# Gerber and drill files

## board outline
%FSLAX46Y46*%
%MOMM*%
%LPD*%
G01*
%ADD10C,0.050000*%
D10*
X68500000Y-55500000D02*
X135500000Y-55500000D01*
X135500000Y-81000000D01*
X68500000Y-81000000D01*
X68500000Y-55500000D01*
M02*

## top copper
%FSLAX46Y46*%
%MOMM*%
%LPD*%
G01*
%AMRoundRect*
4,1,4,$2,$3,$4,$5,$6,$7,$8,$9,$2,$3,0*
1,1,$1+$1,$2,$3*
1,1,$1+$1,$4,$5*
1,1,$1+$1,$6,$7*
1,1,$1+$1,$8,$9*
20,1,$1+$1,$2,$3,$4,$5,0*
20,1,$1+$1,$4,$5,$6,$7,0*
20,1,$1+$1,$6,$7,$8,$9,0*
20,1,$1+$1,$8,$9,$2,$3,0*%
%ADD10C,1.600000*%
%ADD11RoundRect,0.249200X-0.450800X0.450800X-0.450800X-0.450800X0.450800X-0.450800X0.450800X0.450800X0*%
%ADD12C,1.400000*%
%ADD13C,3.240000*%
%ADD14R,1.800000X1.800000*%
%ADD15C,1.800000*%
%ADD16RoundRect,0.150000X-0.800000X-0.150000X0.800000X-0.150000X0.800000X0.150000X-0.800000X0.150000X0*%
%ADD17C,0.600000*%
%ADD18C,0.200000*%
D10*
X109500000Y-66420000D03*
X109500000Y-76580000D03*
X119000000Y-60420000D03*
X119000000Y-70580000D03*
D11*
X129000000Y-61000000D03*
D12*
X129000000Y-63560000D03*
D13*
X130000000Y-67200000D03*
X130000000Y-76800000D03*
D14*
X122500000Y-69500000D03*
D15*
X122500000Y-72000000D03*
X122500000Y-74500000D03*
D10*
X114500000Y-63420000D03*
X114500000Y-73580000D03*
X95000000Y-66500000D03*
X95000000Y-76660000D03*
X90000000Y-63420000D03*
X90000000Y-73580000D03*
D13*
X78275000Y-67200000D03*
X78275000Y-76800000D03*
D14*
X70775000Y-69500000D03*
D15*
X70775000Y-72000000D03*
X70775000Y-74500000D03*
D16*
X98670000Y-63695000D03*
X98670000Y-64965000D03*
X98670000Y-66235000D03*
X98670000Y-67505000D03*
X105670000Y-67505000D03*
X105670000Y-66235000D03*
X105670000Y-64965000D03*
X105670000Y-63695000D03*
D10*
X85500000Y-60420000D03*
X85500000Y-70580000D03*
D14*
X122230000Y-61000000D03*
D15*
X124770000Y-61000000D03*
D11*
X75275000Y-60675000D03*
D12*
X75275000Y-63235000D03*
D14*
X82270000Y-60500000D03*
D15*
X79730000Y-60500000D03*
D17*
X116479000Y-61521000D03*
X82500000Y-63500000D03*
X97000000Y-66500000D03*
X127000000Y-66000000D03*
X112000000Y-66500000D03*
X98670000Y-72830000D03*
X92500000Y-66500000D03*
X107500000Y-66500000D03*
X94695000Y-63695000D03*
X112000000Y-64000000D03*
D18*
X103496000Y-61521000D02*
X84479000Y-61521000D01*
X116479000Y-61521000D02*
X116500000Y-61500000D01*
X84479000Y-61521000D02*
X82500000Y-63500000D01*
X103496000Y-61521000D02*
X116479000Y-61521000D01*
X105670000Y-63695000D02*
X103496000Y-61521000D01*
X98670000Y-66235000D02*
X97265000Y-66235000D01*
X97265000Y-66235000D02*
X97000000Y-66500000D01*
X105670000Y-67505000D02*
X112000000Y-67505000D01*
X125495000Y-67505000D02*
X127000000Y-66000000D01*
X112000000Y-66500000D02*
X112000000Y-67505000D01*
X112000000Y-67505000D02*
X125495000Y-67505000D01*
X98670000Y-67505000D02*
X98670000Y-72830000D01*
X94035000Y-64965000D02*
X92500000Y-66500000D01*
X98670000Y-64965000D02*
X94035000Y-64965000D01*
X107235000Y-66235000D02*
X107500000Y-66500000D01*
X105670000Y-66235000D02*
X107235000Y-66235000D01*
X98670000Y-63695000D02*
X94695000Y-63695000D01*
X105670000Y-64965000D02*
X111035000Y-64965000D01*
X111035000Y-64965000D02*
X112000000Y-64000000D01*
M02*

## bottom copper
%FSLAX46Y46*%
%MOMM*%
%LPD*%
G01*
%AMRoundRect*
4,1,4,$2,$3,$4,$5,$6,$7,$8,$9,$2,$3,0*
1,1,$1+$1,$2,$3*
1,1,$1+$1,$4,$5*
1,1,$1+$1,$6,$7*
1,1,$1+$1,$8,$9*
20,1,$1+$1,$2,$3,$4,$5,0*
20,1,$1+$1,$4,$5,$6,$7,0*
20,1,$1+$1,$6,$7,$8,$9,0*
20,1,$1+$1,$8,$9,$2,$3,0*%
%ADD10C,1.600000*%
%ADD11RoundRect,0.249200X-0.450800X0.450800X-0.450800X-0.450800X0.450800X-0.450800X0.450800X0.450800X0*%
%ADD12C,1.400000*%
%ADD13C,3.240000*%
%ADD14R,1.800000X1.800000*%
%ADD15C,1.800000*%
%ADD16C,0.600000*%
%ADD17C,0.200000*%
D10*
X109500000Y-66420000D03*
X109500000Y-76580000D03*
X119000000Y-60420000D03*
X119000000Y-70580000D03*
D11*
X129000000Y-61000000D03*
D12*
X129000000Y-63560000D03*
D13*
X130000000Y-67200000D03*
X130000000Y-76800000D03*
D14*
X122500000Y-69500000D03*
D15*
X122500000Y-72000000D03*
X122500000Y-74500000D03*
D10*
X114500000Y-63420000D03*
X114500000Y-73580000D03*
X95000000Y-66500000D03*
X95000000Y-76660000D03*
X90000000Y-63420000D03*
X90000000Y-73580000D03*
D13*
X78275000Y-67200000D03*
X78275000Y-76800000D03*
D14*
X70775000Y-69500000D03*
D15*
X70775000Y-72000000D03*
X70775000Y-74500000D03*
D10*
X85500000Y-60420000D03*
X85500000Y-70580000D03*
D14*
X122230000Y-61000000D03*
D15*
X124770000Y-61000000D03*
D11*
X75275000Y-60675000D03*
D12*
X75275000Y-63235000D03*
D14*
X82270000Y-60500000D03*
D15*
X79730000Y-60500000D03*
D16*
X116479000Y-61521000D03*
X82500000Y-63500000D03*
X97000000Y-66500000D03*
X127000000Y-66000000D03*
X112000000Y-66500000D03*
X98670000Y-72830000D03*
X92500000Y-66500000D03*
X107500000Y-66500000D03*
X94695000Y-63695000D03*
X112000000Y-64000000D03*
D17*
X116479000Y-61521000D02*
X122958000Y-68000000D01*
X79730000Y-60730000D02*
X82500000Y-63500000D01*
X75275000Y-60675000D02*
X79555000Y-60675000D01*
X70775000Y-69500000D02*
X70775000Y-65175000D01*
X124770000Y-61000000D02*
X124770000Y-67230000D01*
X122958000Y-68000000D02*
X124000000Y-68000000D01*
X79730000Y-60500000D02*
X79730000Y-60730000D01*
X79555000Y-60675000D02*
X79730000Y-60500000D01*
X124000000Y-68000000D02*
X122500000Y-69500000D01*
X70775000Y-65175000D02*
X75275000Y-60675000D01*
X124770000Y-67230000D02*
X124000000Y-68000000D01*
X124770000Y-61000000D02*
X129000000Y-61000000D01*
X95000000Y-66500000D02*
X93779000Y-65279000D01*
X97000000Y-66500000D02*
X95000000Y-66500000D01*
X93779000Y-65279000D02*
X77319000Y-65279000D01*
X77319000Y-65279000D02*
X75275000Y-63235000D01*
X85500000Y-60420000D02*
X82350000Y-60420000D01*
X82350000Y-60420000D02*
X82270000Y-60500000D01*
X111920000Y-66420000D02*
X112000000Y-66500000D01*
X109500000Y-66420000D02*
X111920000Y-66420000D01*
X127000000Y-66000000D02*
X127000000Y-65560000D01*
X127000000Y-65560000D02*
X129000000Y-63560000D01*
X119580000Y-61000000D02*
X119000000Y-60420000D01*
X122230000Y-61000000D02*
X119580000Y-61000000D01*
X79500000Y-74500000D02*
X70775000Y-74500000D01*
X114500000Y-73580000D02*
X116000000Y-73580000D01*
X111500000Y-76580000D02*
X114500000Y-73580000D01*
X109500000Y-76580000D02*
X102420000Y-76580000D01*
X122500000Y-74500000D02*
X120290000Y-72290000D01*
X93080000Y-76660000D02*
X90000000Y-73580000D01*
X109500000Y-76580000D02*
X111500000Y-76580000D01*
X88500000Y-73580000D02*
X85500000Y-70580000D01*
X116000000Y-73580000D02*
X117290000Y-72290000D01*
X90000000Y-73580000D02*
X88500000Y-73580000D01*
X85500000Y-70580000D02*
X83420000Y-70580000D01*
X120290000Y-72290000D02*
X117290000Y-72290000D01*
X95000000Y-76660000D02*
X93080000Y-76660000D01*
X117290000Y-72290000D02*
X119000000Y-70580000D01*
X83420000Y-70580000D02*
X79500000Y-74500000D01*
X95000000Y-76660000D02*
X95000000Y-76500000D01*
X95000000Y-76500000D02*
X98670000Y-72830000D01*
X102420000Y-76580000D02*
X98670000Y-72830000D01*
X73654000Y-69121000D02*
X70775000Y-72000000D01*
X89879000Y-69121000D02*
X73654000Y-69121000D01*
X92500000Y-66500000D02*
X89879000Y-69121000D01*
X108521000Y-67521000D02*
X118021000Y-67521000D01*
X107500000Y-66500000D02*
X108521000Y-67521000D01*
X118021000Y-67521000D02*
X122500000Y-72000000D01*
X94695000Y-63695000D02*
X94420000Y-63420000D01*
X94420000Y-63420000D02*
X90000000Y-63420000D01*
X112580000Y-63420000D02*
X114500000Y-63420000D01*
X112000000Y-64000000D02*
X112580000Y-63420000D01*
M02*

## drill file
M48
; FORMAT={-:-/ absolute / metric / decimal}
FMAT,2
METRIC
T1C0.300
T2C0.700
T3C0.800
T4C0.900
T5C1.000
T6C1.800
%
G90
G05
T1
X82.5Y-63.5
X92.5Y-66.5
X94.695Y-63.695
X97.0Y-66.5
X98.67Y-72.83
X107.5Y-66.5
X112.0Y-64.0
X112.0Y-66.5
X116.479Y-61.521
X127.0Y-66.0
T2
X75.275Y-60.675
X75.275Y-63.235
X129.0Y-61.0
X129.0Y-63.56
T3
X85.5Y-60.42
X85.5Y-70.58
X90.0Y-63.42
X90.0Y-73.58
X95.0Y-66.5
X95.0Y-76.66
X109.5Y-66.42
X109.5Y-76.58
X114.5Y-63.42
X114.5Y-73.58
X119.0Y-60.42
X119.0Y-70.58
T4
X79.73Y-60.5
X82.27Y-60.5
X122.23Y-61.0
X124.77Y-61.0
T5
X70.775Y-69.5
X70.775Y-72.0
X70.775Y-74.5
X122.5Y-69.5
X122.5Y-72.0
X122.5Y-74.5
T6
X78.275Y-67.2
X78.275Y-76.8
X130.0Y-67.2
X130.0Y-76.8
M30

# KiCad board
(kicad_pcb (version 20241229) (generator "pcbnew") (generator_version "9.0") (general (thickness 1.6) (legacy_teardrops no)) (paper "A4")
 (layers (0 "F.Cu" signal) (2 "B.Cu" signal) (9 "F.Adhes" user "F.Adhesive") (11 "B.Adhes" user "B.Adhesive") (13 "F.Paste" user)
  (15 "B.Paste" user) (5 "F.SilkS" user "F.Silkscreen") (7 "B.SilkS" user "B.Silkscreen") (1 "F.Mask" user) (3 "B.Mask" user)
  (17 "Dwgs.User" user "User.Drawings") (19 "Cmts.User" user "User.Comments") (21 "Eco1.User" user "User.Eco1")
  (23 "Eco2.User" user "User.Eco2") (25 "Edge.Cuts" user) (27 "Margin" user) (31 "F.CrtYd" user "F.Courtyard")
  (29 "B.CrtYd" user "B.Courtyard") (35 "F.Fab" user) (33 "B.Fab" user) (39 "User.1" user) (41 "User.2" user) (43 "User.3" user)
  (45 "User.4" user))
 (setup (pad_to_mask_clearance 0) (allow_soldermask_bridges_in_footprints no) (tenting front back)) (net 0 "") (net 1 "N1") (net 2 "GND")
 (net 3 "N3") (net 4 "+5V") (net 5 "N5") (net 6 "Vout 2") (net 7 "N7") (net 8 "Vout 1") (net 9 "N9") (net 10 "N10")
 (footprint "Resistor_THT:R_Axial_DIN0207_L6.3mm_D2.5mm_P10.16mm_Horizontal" (layer "F.Cu") (at 109.5 66.42 -90)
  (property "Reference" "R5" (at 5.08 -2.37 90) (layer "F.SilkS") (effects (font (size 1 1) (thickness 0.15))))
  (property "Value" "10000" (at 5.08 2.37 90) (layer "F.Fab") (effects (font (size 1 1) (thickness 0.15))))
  (pad "1" thru_hole circle (at 0 0 270) (size 1.6 1.6) (drill 0.8) (layers "*.Cu" "*.Mask") (remove_unused_layers no) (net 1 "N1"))
  (pad "2" thru_hole circle (at 10.16 0 270) (size 1.6 1.6) (drill 0.8) (layers "*.Cu" "*.Mask") (remove_unused_layers no) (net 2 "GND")))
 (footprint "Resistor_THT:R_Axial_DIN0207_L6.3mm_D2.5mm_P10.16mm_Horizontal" (layer "F.Cu") (at 119 60.42 -90)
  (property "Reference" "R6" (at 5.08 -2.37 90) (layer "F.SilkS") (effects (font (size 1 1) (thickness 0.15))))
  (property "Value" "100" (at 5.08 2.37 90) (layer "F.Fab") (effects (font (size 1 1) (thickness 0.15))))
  (pad "1" thru_hole circle (at 0 0 270) (size 1.6 1.6) (drill 0.8) (layers "*.Cu" "*.Mask") (remove_unused_layers no) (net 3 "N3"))
  (pad "2" thru_hole circle (at 10.16 0 270) (size 1.6 1.6) (drill 0.8) (layers "*.Cu" "*.Mask") (remove_unused_layers no) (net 2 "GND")))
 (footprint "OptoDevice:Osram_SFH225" (layer "F.Cu") (at 129 61 -90)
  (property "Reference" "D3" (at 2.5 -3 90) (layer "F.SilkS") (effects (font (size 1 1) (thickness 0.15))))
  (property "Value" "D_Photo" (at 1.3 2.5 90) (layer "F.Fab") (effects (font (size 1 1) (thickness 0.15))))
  (pad "1" thru_hole roundrect (at 0 0 270) (size 1.4 1.4) (drill 0.7) (layers "*.Cu" "*.Mask") (remove_unused_layers no)
   (roundrect_rratio 0.178) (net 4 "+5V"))
  (pad "2" thru_hole circle (at 2.56 0 270) (size 1.4 1.4) (drill 0.7) (layers "*.Cu" "*.Mask") (remove_unused_layers no) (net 1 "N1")))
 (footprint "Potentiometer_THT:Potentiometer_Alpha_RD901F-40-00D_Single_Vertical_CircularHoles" (layer "F.Cu") (at 122.5 69.5)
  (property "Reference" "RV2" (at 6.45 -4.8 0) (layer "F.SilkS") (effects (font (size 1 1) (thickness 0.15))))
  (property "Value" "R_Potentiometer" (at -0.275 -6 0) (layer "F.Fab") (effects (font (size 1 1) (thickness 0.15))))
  (pad "" thru_hole circle (at 7.5 -2.3 90) (size 3.24 3.24) (drill 1.8) (layers "*.Cu" "*.Mask") (remove_unused_layers no))
  (pad "" thru_hole circle (at 7.5 7.3 90) (size 3.24 3.24) (drill 1.8) (layers "*.Cu" "*.Mask") (remove_unused_layers no))
  (pad "1" thru_hole rect (at 0 0 90) (size 1.8 1.8) (drill 1) (layers "*.Cu" "*.Mask") (remove_unused_layers no) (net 4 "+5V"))
  (pad "2" thru_hole circle (at 0 2.5 90) (size 1.8 1.8) (drill 1) (layers "*.Cu" "*.Mask") (remove_unused_layers no) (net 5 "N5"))
  (pad "3" thru_hole circle (at 0 5 90) (size 1.8 1.8) (drill 1) (layers "*.Cu" "*.Mask") (remove_unused_layers no) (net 2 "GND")))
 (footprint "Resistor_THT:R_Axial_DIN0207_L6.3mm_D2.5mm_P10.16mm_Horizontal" (layer "F.Cu") (at 114.5 63.42 -90)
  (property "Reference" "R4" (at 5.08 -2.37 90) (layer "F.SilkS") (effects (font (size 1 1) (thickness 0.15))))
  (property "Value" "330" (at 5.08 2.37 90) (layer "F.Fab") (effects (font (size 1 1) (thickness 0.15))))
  (pad "1" thru_hole circle (at 0 0 270) (size 1.6 1.6) (drill 0.8) (layers "*.Cu" "*.Mask") (remove_unused_layers no) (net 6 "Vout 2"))
  (pad "2" thru_hole circle (at 10.16 0 270) (size 1.6 1.6) (drill 0.8) (layers "*.Cu" "*.Mask") (remove_unused_layers no) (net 2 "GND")))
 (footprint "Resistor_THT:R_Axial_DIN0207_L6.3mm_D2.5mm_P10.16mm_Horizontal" (layer "F.Cu") (at 95 66.5 -90)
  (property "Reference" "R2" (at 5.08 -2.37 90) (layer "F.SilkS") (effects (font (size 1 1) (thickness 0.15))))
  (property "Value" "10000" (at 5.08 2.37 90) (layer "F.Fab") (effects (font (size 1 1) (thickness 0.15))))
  (pad "1" thru_hole circle (at 0 0 270) (size 1.6 1.6) (drill 0.8) (layers "*.Cu" "*.Mask") (remove_unused_layers no) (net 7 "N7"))
  (pad "2" thru_hole circle (at 10.16 0 270) (size 1.6 1.6) (drill 0.8) (layers "*.Cu" "*.Mask") (remove_unused_layers no) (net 2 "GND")))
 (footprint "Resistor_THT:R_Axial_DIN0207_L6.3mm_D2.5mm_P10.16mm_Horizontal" (layer "F.Cu") (at 90 63.42 -90)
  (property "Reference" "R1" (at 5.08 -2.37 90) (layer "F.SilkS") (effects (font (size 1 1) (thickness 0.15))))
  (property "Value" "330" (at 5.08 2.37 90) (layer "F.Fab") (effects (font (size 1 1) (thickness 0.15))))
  (pad "1" thru_hole circle (at 0 0 270) (size 1.6 1.6) (drill 0.8) (layers "*.Cu" "*.Mask") (remove_unused_layers no) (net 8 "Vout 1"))
  (pad "2" thru_hole circle (at 10.16 0 270) (size 1.6 1.6) (drill 0.8) (layers "*.Cu" "*.Mask") (remove_unused_layers no) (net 2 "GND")))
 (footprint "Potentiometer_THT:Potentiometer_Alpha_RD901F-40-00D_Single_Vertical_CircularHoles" (layer "F.Cu") (at 70.775 69.5)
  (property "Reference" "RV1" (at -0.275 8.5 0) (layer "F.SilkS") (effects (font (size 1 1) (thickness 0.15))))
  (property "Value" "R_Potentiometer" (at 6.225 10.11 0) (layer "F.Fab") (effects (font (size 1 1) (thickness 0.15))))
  (pad "" thru_hole circle (at 7.5 -2.3 90) (size 3.24 3.24) (drill 1.8) (layers "*.Cu" "*.Mask") (remove_unused_layers no))
  (pad "" thru_hole circle (at 7.5 7.3 90) (size 3.24 3.24) (drill 1.8) (layers "*.Cu" "*.Mask") (remove_unused_layers no))
  (pad "1" thru_hole rect (at 0 0 90) (size 1.8 1.8) (drill 1) (layers "*.Cu" "*.Mask") (remove_unused_layers no) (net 4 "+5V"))
  (pad "2" thru_hole circle (at 0 2.5 90) (size 1.8 1.8) (drill 1) (layers "*.Cu" "*.Mask") (remove_unused_layers no) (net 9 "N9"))
  (pad "3" thru_hole circle (at 0 5 90) (size 1.8 1.8) (drill 1) (layers "*.Cu" "*.Mask") (remove_unused_layers no) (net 2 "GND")))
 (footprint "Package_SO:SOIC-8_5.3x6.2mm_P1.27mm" (layer "F.Cu") (at 102.17 65.6)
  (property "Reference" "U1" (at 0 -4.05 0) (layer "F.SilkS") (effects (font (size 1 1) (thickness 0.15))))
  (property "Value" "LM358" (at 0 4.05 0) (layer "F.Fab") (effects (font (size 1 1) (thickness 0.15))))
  (pad "1" smd roundrect (at -3.5 -1.905) (size 1.9 0.6) (layers "F.Cu" "F.Mask" "F.Paste") (roundrect_rratio 0.25) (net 8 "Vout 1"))
  (pad "2" smd roundrect (at -3.5 -0.635) (size 1.9 0.6) (layers "F.Cu" "F.Mask" "F.Paste") (roundrect_rratio 0.25) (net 9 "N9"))
  (pad "3" smd roundrect (at -3.5 0.635) (size 1.9 0.6) (layers "F.Cu" "F.Mask" "F.Paste") (roundrect_rratio 0.25) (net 7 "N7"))
  (pad "4" smd roundrect (at -3.5 1.905) (size 1.9 0.6) (layers "F.Cu" "F.Mask" "F.Paste") (roundrect_rratio 0.25) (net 2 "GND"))
  (pad "5" smd roundrect (at 3.5 1.905) (size 1.9 0.6) (layers "F.Cu" "F.Mask" "F.Paste") (roundrect_rratio 0.25) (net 1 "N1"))
  (pad "6" smd roundrect (at 3.5 0.635) (size 1.9 0.6) (layers "F.Cu" "F.Mask" "F.Paste") (roundrect_rratio 0.25) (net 5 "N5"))
  (pad "7" smd roundrect (at 3.5 -0.635) (size 1.9 0.6) (layers "F.Cu" "F.Mask" "F.Paste") (roundrect_rratio 0.25) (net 6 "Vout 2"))
  (pad "8" smd roundrect (at 3.5 -1.905) (size 1.9 0.6) (layers "F.Cu" "F.Mask" "F.Paste") (roundrect_rratio 0.25) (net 4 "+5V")))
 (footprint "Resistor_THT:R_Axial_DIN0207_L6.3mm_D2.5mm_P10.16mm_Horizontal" (layer "F.Cu") (at 85.5 60.42 -90)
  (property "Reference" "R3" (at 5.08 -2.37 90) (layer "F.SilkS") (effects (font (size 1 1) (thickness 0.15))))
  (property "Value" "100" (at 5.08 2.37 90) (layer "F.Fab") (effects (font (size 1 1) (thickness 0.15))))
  (pad "1" thru_hole circle (at 0 0 270) (size 1.6 1.6) (drill 0.8) (layers "*.Cu" "*.Mask") (remove_unused_layers no) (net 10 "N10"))
  (pad "2" thru_hole circle (at 10.16 0 270) (size 1.6 1.6) (drill 0.8) (layers "*.Cu" "*.Mask") (remove_unused_layers no) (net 2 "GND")))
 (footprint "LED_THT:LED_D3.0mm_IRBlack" (layer "F.Cu") (at 122.23 61)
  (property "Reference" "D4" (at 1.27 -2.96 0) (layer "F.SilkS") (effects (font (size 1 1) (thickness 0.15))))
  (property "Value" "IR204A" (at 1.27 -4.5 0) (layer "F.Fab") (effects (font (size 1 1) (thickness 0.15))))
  (pad "1" thru_hole rect (at 0 0) (size 1.8 1.8) (drill 0.9) (layers "*.Cu" "*.Mask") (remove_unused_layers no) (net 3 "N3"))
  (pad "2" thru_hole circle (at 2.54 0) (size 1.8 1.8) (drill 0.9) (layers "*.Cu" "*.Mask") (remove_unused_layers no) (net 4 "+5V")))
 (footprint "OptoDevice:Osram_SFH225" (layer "F.Cu") (at 75.275 60.675 -90)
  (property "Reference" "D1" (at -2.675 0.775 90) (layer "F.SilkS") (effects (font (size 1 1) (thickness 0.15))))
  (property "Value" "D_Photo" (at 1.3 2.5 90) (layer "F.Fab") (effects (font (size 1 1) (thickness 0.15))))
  (pad "1" thru_hole roundrect (at 0 0 270) (size 1.4 1.4) (drill 0.7) (layers "*.Cu" "*.Mask") (remove_unused_layers no)
   (roundrect_rratio 0.178) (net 4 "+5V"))
  (pad "2" thru_hole circle (at 2.56 0 270) (size 1.4 1.4) (drill 0.7) (layers "*.Cu" "*.Mask") (remove_unused_layers no) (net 7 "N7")))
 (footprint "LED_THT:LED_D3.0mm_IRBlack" (layer "F.Cu") (at 82.27 60.5 180)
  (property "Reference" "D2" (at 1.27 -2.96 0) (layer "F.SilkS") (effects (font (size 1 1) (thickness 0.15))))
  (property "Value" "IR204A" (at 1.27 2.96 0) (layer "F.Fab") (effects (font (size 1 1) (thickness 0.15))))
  (pad "1" thru_hole rect (at 0 0 180) (size 1.8 1.8) (drill 0.9) (layers "*.Cu" "*.Mask") (remove_unused_layers no) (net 10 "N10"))
  (pad "2" thru_hole circle (at 2.54 0 180) (size 1.8 1.8) (drill 0.9) (layers "*.Cu" "*.Mask") (remove_unused_layers no) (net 4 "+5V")))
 (gr_rect (start 68.5 55.5) (end 135.5 81) (stroke (width 0.05) (type default)) (fill no) (layer "Edge.Cuts"))
 (segment (start 103.496 61.521) (end 84.479 61.521) (width 0.2) (layer "F.Cu") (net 4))
 (segment (start 116.479 61.521) (end 116.5 61.5) (width 0.2) (layer "F.Cu") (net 4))
 (segment (start 84.479 61.521) (end 82.5 63.5) (width 0.2) (layer "F.Cu") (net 4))
 (segment (start 103.496 61.521) (end 116.479 61.521) (width 0.2) (layer "F.Cu") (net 4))
 (segment (start 105.67 63.695) (end 103.496 61.521) (width 0.2) (layer "F.Cu") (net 4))
 (via (at 116.479 61.521) (size 0.6) (drill 0.3) (layers "F.Cu" "B.Cu") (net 4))
 (via (at 82.5 63.5) (size 0.6) (drill 0.3) (layers "F.Cu" "B.Cu") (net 4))
 (segment (start 116.479 61.521) (end 122.958 68) (width 0.2) (layer "B.Cu") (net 4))
 (segment (start 79.73 60.73) (end 82.5 63.5) (width 0.2) (layer "B.Cu") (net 4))
 (segment (start 75.275 60.675) (end 79.555 60.675) (width 0.2) (layer "B.Cu") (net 4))
 (segment (start 70.775 69.5) (end 70.775 65.175) (width 0.2) (layer "B.Cu") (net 4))
 (segment (start 124.77 61) (end 124.77 67.23) (width 0.2) (layer "B.Cu") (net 4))
 (segment (start 122.958 68) (end 124 68) (width 0.2) (layer "B.Cu") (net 4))
 (segment (start 79.73 60.5) (end 79.73 60.73) (width 0.2) (layer "B.Cu") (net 4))
 (segment (start 79.555 60.675) (end 79.73 60.5) (width 0.2) (layer "B.Cu") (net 4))
 (segment (start 124 68) (end 122.5 69.5) (width 0.2) (layer "B.Cu") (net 4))
 (segment (start 70.775 65.175) (end 75.275 60.675) (width 0.2) (layer "B.Cu") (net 4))
 (segment (start 124.77 67.23) (end 124 68) (width 0.2) (layer "B.Cu") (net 4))
 (segment (start 124.77 61) (end 129 61) (width 0.2) (layer "B.Cu") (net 4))
 (segment (start 98.67 66.235) (end 97.265 66.235) (width 0.2) (layer "F.Cu") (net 7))
 (segment (start 97.265 66.235) (end 97 66.5) (width 0.2) (layer "F.Cu") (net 7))
 (via (at 97 66.5) (size 0.6) (drill 0.3) (layers "F.Cu" "B.Cu") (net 7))
 (segment (start 95 66.5) (end 93.779 65.279) (width 0.2) (layer "B.Cu") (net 7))
 (segment (start 97 66.5) (end 95 66.5) (width 0.2) (layer "B.Cu") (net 7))
 (segment (start 93.779 65.279) (end 77.319 65.279) (width 0.2) (layer "B.Cu") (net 7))
 (segment (start 77.319 65.279) (end 75.275 63.235) (width 0.2) (layer "B.Cu") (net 7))
 (segment (start 85.5 60.42) (end 82.35 60.42) (width 0.2) (layer "B.Cu") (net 10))
 (segment (start 82.35 60.42) (end 82.27 60.5) (width 0.2) (layer "B.Cu") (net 10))
 (segment (start 105.67 67.505) (end 112 67.505) (width 0.2) (layer "F.Cu") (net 1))
 (segment (start 125.495 67.505) (end 127 66) (width 0.2) (layer "F.Cu") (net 1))
 (segment (start 112 66.5) (end 112 67.505) (width 0.2) (layer "F.Cu") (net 1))
 (segment (start 112 67.505) (end 125.495 67.505) (width 0.2) (layer "F.Cu") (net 1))
 (via (at 127 66) (size 0.6) (drill 0.3) (layers "F.Cu" "B.Cu") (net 1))
 (via (at 112 66.5) (size 0.6) (drill 0.3) (layers "F.Cu" "B.Cu") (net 1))
 (segment (start 111.92 66.42) (end 112 66.5) (width 0.2) (layer "B.Cu") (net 1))
 (segment (start 109.5 66.42) (end 111.92 66.42) (width 0.2) (layer "B.Cu") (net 1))
 (segment (start 127 66) (end 127 65.56) (width 0.2) (layer "B.Cu") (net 1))
 (segment (start 127 65.56) (end 129 63.56) (width 0.2) (layer "B.Cu") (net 1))
 (segment (start 119.58 61) (end 119 60.42) (width 0.2) (layer "B.Cu") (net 3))
 (segment (start 122.23 61) (end 119.58 61) (width 0.2) (layer "B.Cu") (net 3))
 (segment (start 98.67 67.505) (end 98.67 72.83) (width 0.2) (layer "F.Cu") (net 2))
 (via (at 98.67 72.83) (size 0.6) (drill 0.3) (layers "F.Cu" "B.Cu") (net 2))
 (segment (start 79.5 74.5) (end 70.775 74.5) (width 0.2) (layer "B.Cu") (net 2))
 (segment (start 114.5 73.58) (end 116 73.58) (width 0.2) (layer "B.Cu") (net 2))
 (segment (start 111.5 76.58) (end 114.5 73.58) (width 0.2) (layer "B.Cu") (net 2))
 (segment (start 109.5 76.58) (end 102.42 76.58) (width 0.2) (layer "B.Cu") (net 2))
 (segment (start 122.5 74.5) (end 120.29 72.29) (width 0.2) (layer "B.Cu") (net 2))
 (segment (start 93.08 76.66) (end 90 73.58) (width 0.2) (layer "B.Cu") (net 2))
 (segment (start 109.5 76.58) (end 111.5 76.58) (width 0.2) (layer "B.Cu") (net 2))
 (segment (start 88.5 73.58) (end 85.5 70.58) (width 0.2) (layer "B.Cu") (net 2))
 (segment (start 116 73.58) (end 117.29 72.29) (width 0.2) (layer "B.Cu") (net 2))
 (segment (start 90 73.58) (end 88.5 73.58) (width 0.2) (layer "B.Cu") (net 2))
 (segment (start 85.5 70.58) (end 83.42 70.58) (width 0.2) (layer "B.Cu") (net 2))
 (segment (start 120.29 72.29) (end 117.29 72.29) (width 0.2) (layer "B.Cu") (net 2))
 (segment (start 95 76.66) (end 93.08 76.66) (width 0.2) (layer "B.Cu") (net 2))
 (segment (start 117.29 72.29) (end 119 70.58) (width 0.2) (layer "B.Cu") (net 2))
 (segment (start 83.42 70.58) (end 79.5 74.5) (width 0.2) (layer "B.Cu") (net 2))
 (segment (start 95 76.66) (end 95 76.5) (width 0.2) (layer "B.Cu") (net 2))
 (segment (start 95 76.5) (end 98.67 72.83) (width 0.2) (layer "B.Cu") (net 2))
 (segment (start 102.42 76.58) (end 98.67 72.83) (width 0.2) (layer "B.Cu") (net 2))
 (segment (start 94.035 64.965) (end 92.5 66.5) (width 0.2) (layer "F.Cu") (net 9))
 (segment (start 98.67 64.965) (end 94.035 64.965) (width 0.2) (layer "F.Cu") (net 9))
 (via (at 92.5 66.5) (size 0.6) (drill 0.3) (layers "F.Cu" "B.Cu") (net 9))
 (segment (start 73.654 69.121) (end 70.775 72) (width 0.2) (layer "B.Cu") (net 9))
 (segment (start 89.879 69.121) (end 73.654 69.121) (width 0.2) (layer "B.Cu") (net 9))
 (segment (start 92.5 66.5) (end 89.879 69.121) (width 0.2) (layer "B.Cu") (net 9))
 (segment (start 107.235 66.235) (end 107.5 66.5) (width 0.2) (layer "F.Cu") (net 5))
 (segment (start 105.67 66.235) (end 107.235 66.235) (width 0.2) (layer "F.Cu") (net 5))
 (via (at 107.5 66.5) (size 0.6) (drill 0.3) (layers "F.Cu" "B.Cu") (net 5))
 (segment (start 108.521 67.521) (end 118.021 67.521) (width 0.2) (layer "B.Cu") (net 5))
 (segment (start 107.5 66.5) (end 108.521 67.521) (width 0.2) (layer "B.Cu") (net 5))
 (segment (start 118.021 67.521) (end 122.5 72) (width 0.2) (layer "B.Cu") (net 5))
 (segment (start 98.67 63.695) (end 94.695 63.695) (width 0.2) (layer "F.Cu") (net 8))
 (via (at 94.695 63.695) (size 0.6) (drill 0.3) (layers "F.Cu" "B.Cu") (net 8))
 (segment (start 94.695 63.695) (end 94.42 63.42) (width 0.2) (layer "B.Cu") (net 8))
 (segment (start 94.42 63.42) (end 90 63.42) (width 0.2) (layer "B.Cu") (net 8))
 (segment (start 105.67 64.965) (end 111.035 64.965) (width 0.2) (layer "F.Cu") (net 6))
 (segment (start 111.035 64.965) (end 112 64) (width 0.2) (layer "F.Cu") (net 6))
 (via (at 112 64) (size 0.6) (drill 0.3) (layers "F.Cu" "B.Cu") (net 6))
 (segment (start 112.58 63.42) (end 114.5 63.42) (width 0.2) (layer "B.Cu") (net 6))
 (segment (start 112 64) (end 112.58 63.42) (width 0.2) (layer "B.Cu") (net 6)))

